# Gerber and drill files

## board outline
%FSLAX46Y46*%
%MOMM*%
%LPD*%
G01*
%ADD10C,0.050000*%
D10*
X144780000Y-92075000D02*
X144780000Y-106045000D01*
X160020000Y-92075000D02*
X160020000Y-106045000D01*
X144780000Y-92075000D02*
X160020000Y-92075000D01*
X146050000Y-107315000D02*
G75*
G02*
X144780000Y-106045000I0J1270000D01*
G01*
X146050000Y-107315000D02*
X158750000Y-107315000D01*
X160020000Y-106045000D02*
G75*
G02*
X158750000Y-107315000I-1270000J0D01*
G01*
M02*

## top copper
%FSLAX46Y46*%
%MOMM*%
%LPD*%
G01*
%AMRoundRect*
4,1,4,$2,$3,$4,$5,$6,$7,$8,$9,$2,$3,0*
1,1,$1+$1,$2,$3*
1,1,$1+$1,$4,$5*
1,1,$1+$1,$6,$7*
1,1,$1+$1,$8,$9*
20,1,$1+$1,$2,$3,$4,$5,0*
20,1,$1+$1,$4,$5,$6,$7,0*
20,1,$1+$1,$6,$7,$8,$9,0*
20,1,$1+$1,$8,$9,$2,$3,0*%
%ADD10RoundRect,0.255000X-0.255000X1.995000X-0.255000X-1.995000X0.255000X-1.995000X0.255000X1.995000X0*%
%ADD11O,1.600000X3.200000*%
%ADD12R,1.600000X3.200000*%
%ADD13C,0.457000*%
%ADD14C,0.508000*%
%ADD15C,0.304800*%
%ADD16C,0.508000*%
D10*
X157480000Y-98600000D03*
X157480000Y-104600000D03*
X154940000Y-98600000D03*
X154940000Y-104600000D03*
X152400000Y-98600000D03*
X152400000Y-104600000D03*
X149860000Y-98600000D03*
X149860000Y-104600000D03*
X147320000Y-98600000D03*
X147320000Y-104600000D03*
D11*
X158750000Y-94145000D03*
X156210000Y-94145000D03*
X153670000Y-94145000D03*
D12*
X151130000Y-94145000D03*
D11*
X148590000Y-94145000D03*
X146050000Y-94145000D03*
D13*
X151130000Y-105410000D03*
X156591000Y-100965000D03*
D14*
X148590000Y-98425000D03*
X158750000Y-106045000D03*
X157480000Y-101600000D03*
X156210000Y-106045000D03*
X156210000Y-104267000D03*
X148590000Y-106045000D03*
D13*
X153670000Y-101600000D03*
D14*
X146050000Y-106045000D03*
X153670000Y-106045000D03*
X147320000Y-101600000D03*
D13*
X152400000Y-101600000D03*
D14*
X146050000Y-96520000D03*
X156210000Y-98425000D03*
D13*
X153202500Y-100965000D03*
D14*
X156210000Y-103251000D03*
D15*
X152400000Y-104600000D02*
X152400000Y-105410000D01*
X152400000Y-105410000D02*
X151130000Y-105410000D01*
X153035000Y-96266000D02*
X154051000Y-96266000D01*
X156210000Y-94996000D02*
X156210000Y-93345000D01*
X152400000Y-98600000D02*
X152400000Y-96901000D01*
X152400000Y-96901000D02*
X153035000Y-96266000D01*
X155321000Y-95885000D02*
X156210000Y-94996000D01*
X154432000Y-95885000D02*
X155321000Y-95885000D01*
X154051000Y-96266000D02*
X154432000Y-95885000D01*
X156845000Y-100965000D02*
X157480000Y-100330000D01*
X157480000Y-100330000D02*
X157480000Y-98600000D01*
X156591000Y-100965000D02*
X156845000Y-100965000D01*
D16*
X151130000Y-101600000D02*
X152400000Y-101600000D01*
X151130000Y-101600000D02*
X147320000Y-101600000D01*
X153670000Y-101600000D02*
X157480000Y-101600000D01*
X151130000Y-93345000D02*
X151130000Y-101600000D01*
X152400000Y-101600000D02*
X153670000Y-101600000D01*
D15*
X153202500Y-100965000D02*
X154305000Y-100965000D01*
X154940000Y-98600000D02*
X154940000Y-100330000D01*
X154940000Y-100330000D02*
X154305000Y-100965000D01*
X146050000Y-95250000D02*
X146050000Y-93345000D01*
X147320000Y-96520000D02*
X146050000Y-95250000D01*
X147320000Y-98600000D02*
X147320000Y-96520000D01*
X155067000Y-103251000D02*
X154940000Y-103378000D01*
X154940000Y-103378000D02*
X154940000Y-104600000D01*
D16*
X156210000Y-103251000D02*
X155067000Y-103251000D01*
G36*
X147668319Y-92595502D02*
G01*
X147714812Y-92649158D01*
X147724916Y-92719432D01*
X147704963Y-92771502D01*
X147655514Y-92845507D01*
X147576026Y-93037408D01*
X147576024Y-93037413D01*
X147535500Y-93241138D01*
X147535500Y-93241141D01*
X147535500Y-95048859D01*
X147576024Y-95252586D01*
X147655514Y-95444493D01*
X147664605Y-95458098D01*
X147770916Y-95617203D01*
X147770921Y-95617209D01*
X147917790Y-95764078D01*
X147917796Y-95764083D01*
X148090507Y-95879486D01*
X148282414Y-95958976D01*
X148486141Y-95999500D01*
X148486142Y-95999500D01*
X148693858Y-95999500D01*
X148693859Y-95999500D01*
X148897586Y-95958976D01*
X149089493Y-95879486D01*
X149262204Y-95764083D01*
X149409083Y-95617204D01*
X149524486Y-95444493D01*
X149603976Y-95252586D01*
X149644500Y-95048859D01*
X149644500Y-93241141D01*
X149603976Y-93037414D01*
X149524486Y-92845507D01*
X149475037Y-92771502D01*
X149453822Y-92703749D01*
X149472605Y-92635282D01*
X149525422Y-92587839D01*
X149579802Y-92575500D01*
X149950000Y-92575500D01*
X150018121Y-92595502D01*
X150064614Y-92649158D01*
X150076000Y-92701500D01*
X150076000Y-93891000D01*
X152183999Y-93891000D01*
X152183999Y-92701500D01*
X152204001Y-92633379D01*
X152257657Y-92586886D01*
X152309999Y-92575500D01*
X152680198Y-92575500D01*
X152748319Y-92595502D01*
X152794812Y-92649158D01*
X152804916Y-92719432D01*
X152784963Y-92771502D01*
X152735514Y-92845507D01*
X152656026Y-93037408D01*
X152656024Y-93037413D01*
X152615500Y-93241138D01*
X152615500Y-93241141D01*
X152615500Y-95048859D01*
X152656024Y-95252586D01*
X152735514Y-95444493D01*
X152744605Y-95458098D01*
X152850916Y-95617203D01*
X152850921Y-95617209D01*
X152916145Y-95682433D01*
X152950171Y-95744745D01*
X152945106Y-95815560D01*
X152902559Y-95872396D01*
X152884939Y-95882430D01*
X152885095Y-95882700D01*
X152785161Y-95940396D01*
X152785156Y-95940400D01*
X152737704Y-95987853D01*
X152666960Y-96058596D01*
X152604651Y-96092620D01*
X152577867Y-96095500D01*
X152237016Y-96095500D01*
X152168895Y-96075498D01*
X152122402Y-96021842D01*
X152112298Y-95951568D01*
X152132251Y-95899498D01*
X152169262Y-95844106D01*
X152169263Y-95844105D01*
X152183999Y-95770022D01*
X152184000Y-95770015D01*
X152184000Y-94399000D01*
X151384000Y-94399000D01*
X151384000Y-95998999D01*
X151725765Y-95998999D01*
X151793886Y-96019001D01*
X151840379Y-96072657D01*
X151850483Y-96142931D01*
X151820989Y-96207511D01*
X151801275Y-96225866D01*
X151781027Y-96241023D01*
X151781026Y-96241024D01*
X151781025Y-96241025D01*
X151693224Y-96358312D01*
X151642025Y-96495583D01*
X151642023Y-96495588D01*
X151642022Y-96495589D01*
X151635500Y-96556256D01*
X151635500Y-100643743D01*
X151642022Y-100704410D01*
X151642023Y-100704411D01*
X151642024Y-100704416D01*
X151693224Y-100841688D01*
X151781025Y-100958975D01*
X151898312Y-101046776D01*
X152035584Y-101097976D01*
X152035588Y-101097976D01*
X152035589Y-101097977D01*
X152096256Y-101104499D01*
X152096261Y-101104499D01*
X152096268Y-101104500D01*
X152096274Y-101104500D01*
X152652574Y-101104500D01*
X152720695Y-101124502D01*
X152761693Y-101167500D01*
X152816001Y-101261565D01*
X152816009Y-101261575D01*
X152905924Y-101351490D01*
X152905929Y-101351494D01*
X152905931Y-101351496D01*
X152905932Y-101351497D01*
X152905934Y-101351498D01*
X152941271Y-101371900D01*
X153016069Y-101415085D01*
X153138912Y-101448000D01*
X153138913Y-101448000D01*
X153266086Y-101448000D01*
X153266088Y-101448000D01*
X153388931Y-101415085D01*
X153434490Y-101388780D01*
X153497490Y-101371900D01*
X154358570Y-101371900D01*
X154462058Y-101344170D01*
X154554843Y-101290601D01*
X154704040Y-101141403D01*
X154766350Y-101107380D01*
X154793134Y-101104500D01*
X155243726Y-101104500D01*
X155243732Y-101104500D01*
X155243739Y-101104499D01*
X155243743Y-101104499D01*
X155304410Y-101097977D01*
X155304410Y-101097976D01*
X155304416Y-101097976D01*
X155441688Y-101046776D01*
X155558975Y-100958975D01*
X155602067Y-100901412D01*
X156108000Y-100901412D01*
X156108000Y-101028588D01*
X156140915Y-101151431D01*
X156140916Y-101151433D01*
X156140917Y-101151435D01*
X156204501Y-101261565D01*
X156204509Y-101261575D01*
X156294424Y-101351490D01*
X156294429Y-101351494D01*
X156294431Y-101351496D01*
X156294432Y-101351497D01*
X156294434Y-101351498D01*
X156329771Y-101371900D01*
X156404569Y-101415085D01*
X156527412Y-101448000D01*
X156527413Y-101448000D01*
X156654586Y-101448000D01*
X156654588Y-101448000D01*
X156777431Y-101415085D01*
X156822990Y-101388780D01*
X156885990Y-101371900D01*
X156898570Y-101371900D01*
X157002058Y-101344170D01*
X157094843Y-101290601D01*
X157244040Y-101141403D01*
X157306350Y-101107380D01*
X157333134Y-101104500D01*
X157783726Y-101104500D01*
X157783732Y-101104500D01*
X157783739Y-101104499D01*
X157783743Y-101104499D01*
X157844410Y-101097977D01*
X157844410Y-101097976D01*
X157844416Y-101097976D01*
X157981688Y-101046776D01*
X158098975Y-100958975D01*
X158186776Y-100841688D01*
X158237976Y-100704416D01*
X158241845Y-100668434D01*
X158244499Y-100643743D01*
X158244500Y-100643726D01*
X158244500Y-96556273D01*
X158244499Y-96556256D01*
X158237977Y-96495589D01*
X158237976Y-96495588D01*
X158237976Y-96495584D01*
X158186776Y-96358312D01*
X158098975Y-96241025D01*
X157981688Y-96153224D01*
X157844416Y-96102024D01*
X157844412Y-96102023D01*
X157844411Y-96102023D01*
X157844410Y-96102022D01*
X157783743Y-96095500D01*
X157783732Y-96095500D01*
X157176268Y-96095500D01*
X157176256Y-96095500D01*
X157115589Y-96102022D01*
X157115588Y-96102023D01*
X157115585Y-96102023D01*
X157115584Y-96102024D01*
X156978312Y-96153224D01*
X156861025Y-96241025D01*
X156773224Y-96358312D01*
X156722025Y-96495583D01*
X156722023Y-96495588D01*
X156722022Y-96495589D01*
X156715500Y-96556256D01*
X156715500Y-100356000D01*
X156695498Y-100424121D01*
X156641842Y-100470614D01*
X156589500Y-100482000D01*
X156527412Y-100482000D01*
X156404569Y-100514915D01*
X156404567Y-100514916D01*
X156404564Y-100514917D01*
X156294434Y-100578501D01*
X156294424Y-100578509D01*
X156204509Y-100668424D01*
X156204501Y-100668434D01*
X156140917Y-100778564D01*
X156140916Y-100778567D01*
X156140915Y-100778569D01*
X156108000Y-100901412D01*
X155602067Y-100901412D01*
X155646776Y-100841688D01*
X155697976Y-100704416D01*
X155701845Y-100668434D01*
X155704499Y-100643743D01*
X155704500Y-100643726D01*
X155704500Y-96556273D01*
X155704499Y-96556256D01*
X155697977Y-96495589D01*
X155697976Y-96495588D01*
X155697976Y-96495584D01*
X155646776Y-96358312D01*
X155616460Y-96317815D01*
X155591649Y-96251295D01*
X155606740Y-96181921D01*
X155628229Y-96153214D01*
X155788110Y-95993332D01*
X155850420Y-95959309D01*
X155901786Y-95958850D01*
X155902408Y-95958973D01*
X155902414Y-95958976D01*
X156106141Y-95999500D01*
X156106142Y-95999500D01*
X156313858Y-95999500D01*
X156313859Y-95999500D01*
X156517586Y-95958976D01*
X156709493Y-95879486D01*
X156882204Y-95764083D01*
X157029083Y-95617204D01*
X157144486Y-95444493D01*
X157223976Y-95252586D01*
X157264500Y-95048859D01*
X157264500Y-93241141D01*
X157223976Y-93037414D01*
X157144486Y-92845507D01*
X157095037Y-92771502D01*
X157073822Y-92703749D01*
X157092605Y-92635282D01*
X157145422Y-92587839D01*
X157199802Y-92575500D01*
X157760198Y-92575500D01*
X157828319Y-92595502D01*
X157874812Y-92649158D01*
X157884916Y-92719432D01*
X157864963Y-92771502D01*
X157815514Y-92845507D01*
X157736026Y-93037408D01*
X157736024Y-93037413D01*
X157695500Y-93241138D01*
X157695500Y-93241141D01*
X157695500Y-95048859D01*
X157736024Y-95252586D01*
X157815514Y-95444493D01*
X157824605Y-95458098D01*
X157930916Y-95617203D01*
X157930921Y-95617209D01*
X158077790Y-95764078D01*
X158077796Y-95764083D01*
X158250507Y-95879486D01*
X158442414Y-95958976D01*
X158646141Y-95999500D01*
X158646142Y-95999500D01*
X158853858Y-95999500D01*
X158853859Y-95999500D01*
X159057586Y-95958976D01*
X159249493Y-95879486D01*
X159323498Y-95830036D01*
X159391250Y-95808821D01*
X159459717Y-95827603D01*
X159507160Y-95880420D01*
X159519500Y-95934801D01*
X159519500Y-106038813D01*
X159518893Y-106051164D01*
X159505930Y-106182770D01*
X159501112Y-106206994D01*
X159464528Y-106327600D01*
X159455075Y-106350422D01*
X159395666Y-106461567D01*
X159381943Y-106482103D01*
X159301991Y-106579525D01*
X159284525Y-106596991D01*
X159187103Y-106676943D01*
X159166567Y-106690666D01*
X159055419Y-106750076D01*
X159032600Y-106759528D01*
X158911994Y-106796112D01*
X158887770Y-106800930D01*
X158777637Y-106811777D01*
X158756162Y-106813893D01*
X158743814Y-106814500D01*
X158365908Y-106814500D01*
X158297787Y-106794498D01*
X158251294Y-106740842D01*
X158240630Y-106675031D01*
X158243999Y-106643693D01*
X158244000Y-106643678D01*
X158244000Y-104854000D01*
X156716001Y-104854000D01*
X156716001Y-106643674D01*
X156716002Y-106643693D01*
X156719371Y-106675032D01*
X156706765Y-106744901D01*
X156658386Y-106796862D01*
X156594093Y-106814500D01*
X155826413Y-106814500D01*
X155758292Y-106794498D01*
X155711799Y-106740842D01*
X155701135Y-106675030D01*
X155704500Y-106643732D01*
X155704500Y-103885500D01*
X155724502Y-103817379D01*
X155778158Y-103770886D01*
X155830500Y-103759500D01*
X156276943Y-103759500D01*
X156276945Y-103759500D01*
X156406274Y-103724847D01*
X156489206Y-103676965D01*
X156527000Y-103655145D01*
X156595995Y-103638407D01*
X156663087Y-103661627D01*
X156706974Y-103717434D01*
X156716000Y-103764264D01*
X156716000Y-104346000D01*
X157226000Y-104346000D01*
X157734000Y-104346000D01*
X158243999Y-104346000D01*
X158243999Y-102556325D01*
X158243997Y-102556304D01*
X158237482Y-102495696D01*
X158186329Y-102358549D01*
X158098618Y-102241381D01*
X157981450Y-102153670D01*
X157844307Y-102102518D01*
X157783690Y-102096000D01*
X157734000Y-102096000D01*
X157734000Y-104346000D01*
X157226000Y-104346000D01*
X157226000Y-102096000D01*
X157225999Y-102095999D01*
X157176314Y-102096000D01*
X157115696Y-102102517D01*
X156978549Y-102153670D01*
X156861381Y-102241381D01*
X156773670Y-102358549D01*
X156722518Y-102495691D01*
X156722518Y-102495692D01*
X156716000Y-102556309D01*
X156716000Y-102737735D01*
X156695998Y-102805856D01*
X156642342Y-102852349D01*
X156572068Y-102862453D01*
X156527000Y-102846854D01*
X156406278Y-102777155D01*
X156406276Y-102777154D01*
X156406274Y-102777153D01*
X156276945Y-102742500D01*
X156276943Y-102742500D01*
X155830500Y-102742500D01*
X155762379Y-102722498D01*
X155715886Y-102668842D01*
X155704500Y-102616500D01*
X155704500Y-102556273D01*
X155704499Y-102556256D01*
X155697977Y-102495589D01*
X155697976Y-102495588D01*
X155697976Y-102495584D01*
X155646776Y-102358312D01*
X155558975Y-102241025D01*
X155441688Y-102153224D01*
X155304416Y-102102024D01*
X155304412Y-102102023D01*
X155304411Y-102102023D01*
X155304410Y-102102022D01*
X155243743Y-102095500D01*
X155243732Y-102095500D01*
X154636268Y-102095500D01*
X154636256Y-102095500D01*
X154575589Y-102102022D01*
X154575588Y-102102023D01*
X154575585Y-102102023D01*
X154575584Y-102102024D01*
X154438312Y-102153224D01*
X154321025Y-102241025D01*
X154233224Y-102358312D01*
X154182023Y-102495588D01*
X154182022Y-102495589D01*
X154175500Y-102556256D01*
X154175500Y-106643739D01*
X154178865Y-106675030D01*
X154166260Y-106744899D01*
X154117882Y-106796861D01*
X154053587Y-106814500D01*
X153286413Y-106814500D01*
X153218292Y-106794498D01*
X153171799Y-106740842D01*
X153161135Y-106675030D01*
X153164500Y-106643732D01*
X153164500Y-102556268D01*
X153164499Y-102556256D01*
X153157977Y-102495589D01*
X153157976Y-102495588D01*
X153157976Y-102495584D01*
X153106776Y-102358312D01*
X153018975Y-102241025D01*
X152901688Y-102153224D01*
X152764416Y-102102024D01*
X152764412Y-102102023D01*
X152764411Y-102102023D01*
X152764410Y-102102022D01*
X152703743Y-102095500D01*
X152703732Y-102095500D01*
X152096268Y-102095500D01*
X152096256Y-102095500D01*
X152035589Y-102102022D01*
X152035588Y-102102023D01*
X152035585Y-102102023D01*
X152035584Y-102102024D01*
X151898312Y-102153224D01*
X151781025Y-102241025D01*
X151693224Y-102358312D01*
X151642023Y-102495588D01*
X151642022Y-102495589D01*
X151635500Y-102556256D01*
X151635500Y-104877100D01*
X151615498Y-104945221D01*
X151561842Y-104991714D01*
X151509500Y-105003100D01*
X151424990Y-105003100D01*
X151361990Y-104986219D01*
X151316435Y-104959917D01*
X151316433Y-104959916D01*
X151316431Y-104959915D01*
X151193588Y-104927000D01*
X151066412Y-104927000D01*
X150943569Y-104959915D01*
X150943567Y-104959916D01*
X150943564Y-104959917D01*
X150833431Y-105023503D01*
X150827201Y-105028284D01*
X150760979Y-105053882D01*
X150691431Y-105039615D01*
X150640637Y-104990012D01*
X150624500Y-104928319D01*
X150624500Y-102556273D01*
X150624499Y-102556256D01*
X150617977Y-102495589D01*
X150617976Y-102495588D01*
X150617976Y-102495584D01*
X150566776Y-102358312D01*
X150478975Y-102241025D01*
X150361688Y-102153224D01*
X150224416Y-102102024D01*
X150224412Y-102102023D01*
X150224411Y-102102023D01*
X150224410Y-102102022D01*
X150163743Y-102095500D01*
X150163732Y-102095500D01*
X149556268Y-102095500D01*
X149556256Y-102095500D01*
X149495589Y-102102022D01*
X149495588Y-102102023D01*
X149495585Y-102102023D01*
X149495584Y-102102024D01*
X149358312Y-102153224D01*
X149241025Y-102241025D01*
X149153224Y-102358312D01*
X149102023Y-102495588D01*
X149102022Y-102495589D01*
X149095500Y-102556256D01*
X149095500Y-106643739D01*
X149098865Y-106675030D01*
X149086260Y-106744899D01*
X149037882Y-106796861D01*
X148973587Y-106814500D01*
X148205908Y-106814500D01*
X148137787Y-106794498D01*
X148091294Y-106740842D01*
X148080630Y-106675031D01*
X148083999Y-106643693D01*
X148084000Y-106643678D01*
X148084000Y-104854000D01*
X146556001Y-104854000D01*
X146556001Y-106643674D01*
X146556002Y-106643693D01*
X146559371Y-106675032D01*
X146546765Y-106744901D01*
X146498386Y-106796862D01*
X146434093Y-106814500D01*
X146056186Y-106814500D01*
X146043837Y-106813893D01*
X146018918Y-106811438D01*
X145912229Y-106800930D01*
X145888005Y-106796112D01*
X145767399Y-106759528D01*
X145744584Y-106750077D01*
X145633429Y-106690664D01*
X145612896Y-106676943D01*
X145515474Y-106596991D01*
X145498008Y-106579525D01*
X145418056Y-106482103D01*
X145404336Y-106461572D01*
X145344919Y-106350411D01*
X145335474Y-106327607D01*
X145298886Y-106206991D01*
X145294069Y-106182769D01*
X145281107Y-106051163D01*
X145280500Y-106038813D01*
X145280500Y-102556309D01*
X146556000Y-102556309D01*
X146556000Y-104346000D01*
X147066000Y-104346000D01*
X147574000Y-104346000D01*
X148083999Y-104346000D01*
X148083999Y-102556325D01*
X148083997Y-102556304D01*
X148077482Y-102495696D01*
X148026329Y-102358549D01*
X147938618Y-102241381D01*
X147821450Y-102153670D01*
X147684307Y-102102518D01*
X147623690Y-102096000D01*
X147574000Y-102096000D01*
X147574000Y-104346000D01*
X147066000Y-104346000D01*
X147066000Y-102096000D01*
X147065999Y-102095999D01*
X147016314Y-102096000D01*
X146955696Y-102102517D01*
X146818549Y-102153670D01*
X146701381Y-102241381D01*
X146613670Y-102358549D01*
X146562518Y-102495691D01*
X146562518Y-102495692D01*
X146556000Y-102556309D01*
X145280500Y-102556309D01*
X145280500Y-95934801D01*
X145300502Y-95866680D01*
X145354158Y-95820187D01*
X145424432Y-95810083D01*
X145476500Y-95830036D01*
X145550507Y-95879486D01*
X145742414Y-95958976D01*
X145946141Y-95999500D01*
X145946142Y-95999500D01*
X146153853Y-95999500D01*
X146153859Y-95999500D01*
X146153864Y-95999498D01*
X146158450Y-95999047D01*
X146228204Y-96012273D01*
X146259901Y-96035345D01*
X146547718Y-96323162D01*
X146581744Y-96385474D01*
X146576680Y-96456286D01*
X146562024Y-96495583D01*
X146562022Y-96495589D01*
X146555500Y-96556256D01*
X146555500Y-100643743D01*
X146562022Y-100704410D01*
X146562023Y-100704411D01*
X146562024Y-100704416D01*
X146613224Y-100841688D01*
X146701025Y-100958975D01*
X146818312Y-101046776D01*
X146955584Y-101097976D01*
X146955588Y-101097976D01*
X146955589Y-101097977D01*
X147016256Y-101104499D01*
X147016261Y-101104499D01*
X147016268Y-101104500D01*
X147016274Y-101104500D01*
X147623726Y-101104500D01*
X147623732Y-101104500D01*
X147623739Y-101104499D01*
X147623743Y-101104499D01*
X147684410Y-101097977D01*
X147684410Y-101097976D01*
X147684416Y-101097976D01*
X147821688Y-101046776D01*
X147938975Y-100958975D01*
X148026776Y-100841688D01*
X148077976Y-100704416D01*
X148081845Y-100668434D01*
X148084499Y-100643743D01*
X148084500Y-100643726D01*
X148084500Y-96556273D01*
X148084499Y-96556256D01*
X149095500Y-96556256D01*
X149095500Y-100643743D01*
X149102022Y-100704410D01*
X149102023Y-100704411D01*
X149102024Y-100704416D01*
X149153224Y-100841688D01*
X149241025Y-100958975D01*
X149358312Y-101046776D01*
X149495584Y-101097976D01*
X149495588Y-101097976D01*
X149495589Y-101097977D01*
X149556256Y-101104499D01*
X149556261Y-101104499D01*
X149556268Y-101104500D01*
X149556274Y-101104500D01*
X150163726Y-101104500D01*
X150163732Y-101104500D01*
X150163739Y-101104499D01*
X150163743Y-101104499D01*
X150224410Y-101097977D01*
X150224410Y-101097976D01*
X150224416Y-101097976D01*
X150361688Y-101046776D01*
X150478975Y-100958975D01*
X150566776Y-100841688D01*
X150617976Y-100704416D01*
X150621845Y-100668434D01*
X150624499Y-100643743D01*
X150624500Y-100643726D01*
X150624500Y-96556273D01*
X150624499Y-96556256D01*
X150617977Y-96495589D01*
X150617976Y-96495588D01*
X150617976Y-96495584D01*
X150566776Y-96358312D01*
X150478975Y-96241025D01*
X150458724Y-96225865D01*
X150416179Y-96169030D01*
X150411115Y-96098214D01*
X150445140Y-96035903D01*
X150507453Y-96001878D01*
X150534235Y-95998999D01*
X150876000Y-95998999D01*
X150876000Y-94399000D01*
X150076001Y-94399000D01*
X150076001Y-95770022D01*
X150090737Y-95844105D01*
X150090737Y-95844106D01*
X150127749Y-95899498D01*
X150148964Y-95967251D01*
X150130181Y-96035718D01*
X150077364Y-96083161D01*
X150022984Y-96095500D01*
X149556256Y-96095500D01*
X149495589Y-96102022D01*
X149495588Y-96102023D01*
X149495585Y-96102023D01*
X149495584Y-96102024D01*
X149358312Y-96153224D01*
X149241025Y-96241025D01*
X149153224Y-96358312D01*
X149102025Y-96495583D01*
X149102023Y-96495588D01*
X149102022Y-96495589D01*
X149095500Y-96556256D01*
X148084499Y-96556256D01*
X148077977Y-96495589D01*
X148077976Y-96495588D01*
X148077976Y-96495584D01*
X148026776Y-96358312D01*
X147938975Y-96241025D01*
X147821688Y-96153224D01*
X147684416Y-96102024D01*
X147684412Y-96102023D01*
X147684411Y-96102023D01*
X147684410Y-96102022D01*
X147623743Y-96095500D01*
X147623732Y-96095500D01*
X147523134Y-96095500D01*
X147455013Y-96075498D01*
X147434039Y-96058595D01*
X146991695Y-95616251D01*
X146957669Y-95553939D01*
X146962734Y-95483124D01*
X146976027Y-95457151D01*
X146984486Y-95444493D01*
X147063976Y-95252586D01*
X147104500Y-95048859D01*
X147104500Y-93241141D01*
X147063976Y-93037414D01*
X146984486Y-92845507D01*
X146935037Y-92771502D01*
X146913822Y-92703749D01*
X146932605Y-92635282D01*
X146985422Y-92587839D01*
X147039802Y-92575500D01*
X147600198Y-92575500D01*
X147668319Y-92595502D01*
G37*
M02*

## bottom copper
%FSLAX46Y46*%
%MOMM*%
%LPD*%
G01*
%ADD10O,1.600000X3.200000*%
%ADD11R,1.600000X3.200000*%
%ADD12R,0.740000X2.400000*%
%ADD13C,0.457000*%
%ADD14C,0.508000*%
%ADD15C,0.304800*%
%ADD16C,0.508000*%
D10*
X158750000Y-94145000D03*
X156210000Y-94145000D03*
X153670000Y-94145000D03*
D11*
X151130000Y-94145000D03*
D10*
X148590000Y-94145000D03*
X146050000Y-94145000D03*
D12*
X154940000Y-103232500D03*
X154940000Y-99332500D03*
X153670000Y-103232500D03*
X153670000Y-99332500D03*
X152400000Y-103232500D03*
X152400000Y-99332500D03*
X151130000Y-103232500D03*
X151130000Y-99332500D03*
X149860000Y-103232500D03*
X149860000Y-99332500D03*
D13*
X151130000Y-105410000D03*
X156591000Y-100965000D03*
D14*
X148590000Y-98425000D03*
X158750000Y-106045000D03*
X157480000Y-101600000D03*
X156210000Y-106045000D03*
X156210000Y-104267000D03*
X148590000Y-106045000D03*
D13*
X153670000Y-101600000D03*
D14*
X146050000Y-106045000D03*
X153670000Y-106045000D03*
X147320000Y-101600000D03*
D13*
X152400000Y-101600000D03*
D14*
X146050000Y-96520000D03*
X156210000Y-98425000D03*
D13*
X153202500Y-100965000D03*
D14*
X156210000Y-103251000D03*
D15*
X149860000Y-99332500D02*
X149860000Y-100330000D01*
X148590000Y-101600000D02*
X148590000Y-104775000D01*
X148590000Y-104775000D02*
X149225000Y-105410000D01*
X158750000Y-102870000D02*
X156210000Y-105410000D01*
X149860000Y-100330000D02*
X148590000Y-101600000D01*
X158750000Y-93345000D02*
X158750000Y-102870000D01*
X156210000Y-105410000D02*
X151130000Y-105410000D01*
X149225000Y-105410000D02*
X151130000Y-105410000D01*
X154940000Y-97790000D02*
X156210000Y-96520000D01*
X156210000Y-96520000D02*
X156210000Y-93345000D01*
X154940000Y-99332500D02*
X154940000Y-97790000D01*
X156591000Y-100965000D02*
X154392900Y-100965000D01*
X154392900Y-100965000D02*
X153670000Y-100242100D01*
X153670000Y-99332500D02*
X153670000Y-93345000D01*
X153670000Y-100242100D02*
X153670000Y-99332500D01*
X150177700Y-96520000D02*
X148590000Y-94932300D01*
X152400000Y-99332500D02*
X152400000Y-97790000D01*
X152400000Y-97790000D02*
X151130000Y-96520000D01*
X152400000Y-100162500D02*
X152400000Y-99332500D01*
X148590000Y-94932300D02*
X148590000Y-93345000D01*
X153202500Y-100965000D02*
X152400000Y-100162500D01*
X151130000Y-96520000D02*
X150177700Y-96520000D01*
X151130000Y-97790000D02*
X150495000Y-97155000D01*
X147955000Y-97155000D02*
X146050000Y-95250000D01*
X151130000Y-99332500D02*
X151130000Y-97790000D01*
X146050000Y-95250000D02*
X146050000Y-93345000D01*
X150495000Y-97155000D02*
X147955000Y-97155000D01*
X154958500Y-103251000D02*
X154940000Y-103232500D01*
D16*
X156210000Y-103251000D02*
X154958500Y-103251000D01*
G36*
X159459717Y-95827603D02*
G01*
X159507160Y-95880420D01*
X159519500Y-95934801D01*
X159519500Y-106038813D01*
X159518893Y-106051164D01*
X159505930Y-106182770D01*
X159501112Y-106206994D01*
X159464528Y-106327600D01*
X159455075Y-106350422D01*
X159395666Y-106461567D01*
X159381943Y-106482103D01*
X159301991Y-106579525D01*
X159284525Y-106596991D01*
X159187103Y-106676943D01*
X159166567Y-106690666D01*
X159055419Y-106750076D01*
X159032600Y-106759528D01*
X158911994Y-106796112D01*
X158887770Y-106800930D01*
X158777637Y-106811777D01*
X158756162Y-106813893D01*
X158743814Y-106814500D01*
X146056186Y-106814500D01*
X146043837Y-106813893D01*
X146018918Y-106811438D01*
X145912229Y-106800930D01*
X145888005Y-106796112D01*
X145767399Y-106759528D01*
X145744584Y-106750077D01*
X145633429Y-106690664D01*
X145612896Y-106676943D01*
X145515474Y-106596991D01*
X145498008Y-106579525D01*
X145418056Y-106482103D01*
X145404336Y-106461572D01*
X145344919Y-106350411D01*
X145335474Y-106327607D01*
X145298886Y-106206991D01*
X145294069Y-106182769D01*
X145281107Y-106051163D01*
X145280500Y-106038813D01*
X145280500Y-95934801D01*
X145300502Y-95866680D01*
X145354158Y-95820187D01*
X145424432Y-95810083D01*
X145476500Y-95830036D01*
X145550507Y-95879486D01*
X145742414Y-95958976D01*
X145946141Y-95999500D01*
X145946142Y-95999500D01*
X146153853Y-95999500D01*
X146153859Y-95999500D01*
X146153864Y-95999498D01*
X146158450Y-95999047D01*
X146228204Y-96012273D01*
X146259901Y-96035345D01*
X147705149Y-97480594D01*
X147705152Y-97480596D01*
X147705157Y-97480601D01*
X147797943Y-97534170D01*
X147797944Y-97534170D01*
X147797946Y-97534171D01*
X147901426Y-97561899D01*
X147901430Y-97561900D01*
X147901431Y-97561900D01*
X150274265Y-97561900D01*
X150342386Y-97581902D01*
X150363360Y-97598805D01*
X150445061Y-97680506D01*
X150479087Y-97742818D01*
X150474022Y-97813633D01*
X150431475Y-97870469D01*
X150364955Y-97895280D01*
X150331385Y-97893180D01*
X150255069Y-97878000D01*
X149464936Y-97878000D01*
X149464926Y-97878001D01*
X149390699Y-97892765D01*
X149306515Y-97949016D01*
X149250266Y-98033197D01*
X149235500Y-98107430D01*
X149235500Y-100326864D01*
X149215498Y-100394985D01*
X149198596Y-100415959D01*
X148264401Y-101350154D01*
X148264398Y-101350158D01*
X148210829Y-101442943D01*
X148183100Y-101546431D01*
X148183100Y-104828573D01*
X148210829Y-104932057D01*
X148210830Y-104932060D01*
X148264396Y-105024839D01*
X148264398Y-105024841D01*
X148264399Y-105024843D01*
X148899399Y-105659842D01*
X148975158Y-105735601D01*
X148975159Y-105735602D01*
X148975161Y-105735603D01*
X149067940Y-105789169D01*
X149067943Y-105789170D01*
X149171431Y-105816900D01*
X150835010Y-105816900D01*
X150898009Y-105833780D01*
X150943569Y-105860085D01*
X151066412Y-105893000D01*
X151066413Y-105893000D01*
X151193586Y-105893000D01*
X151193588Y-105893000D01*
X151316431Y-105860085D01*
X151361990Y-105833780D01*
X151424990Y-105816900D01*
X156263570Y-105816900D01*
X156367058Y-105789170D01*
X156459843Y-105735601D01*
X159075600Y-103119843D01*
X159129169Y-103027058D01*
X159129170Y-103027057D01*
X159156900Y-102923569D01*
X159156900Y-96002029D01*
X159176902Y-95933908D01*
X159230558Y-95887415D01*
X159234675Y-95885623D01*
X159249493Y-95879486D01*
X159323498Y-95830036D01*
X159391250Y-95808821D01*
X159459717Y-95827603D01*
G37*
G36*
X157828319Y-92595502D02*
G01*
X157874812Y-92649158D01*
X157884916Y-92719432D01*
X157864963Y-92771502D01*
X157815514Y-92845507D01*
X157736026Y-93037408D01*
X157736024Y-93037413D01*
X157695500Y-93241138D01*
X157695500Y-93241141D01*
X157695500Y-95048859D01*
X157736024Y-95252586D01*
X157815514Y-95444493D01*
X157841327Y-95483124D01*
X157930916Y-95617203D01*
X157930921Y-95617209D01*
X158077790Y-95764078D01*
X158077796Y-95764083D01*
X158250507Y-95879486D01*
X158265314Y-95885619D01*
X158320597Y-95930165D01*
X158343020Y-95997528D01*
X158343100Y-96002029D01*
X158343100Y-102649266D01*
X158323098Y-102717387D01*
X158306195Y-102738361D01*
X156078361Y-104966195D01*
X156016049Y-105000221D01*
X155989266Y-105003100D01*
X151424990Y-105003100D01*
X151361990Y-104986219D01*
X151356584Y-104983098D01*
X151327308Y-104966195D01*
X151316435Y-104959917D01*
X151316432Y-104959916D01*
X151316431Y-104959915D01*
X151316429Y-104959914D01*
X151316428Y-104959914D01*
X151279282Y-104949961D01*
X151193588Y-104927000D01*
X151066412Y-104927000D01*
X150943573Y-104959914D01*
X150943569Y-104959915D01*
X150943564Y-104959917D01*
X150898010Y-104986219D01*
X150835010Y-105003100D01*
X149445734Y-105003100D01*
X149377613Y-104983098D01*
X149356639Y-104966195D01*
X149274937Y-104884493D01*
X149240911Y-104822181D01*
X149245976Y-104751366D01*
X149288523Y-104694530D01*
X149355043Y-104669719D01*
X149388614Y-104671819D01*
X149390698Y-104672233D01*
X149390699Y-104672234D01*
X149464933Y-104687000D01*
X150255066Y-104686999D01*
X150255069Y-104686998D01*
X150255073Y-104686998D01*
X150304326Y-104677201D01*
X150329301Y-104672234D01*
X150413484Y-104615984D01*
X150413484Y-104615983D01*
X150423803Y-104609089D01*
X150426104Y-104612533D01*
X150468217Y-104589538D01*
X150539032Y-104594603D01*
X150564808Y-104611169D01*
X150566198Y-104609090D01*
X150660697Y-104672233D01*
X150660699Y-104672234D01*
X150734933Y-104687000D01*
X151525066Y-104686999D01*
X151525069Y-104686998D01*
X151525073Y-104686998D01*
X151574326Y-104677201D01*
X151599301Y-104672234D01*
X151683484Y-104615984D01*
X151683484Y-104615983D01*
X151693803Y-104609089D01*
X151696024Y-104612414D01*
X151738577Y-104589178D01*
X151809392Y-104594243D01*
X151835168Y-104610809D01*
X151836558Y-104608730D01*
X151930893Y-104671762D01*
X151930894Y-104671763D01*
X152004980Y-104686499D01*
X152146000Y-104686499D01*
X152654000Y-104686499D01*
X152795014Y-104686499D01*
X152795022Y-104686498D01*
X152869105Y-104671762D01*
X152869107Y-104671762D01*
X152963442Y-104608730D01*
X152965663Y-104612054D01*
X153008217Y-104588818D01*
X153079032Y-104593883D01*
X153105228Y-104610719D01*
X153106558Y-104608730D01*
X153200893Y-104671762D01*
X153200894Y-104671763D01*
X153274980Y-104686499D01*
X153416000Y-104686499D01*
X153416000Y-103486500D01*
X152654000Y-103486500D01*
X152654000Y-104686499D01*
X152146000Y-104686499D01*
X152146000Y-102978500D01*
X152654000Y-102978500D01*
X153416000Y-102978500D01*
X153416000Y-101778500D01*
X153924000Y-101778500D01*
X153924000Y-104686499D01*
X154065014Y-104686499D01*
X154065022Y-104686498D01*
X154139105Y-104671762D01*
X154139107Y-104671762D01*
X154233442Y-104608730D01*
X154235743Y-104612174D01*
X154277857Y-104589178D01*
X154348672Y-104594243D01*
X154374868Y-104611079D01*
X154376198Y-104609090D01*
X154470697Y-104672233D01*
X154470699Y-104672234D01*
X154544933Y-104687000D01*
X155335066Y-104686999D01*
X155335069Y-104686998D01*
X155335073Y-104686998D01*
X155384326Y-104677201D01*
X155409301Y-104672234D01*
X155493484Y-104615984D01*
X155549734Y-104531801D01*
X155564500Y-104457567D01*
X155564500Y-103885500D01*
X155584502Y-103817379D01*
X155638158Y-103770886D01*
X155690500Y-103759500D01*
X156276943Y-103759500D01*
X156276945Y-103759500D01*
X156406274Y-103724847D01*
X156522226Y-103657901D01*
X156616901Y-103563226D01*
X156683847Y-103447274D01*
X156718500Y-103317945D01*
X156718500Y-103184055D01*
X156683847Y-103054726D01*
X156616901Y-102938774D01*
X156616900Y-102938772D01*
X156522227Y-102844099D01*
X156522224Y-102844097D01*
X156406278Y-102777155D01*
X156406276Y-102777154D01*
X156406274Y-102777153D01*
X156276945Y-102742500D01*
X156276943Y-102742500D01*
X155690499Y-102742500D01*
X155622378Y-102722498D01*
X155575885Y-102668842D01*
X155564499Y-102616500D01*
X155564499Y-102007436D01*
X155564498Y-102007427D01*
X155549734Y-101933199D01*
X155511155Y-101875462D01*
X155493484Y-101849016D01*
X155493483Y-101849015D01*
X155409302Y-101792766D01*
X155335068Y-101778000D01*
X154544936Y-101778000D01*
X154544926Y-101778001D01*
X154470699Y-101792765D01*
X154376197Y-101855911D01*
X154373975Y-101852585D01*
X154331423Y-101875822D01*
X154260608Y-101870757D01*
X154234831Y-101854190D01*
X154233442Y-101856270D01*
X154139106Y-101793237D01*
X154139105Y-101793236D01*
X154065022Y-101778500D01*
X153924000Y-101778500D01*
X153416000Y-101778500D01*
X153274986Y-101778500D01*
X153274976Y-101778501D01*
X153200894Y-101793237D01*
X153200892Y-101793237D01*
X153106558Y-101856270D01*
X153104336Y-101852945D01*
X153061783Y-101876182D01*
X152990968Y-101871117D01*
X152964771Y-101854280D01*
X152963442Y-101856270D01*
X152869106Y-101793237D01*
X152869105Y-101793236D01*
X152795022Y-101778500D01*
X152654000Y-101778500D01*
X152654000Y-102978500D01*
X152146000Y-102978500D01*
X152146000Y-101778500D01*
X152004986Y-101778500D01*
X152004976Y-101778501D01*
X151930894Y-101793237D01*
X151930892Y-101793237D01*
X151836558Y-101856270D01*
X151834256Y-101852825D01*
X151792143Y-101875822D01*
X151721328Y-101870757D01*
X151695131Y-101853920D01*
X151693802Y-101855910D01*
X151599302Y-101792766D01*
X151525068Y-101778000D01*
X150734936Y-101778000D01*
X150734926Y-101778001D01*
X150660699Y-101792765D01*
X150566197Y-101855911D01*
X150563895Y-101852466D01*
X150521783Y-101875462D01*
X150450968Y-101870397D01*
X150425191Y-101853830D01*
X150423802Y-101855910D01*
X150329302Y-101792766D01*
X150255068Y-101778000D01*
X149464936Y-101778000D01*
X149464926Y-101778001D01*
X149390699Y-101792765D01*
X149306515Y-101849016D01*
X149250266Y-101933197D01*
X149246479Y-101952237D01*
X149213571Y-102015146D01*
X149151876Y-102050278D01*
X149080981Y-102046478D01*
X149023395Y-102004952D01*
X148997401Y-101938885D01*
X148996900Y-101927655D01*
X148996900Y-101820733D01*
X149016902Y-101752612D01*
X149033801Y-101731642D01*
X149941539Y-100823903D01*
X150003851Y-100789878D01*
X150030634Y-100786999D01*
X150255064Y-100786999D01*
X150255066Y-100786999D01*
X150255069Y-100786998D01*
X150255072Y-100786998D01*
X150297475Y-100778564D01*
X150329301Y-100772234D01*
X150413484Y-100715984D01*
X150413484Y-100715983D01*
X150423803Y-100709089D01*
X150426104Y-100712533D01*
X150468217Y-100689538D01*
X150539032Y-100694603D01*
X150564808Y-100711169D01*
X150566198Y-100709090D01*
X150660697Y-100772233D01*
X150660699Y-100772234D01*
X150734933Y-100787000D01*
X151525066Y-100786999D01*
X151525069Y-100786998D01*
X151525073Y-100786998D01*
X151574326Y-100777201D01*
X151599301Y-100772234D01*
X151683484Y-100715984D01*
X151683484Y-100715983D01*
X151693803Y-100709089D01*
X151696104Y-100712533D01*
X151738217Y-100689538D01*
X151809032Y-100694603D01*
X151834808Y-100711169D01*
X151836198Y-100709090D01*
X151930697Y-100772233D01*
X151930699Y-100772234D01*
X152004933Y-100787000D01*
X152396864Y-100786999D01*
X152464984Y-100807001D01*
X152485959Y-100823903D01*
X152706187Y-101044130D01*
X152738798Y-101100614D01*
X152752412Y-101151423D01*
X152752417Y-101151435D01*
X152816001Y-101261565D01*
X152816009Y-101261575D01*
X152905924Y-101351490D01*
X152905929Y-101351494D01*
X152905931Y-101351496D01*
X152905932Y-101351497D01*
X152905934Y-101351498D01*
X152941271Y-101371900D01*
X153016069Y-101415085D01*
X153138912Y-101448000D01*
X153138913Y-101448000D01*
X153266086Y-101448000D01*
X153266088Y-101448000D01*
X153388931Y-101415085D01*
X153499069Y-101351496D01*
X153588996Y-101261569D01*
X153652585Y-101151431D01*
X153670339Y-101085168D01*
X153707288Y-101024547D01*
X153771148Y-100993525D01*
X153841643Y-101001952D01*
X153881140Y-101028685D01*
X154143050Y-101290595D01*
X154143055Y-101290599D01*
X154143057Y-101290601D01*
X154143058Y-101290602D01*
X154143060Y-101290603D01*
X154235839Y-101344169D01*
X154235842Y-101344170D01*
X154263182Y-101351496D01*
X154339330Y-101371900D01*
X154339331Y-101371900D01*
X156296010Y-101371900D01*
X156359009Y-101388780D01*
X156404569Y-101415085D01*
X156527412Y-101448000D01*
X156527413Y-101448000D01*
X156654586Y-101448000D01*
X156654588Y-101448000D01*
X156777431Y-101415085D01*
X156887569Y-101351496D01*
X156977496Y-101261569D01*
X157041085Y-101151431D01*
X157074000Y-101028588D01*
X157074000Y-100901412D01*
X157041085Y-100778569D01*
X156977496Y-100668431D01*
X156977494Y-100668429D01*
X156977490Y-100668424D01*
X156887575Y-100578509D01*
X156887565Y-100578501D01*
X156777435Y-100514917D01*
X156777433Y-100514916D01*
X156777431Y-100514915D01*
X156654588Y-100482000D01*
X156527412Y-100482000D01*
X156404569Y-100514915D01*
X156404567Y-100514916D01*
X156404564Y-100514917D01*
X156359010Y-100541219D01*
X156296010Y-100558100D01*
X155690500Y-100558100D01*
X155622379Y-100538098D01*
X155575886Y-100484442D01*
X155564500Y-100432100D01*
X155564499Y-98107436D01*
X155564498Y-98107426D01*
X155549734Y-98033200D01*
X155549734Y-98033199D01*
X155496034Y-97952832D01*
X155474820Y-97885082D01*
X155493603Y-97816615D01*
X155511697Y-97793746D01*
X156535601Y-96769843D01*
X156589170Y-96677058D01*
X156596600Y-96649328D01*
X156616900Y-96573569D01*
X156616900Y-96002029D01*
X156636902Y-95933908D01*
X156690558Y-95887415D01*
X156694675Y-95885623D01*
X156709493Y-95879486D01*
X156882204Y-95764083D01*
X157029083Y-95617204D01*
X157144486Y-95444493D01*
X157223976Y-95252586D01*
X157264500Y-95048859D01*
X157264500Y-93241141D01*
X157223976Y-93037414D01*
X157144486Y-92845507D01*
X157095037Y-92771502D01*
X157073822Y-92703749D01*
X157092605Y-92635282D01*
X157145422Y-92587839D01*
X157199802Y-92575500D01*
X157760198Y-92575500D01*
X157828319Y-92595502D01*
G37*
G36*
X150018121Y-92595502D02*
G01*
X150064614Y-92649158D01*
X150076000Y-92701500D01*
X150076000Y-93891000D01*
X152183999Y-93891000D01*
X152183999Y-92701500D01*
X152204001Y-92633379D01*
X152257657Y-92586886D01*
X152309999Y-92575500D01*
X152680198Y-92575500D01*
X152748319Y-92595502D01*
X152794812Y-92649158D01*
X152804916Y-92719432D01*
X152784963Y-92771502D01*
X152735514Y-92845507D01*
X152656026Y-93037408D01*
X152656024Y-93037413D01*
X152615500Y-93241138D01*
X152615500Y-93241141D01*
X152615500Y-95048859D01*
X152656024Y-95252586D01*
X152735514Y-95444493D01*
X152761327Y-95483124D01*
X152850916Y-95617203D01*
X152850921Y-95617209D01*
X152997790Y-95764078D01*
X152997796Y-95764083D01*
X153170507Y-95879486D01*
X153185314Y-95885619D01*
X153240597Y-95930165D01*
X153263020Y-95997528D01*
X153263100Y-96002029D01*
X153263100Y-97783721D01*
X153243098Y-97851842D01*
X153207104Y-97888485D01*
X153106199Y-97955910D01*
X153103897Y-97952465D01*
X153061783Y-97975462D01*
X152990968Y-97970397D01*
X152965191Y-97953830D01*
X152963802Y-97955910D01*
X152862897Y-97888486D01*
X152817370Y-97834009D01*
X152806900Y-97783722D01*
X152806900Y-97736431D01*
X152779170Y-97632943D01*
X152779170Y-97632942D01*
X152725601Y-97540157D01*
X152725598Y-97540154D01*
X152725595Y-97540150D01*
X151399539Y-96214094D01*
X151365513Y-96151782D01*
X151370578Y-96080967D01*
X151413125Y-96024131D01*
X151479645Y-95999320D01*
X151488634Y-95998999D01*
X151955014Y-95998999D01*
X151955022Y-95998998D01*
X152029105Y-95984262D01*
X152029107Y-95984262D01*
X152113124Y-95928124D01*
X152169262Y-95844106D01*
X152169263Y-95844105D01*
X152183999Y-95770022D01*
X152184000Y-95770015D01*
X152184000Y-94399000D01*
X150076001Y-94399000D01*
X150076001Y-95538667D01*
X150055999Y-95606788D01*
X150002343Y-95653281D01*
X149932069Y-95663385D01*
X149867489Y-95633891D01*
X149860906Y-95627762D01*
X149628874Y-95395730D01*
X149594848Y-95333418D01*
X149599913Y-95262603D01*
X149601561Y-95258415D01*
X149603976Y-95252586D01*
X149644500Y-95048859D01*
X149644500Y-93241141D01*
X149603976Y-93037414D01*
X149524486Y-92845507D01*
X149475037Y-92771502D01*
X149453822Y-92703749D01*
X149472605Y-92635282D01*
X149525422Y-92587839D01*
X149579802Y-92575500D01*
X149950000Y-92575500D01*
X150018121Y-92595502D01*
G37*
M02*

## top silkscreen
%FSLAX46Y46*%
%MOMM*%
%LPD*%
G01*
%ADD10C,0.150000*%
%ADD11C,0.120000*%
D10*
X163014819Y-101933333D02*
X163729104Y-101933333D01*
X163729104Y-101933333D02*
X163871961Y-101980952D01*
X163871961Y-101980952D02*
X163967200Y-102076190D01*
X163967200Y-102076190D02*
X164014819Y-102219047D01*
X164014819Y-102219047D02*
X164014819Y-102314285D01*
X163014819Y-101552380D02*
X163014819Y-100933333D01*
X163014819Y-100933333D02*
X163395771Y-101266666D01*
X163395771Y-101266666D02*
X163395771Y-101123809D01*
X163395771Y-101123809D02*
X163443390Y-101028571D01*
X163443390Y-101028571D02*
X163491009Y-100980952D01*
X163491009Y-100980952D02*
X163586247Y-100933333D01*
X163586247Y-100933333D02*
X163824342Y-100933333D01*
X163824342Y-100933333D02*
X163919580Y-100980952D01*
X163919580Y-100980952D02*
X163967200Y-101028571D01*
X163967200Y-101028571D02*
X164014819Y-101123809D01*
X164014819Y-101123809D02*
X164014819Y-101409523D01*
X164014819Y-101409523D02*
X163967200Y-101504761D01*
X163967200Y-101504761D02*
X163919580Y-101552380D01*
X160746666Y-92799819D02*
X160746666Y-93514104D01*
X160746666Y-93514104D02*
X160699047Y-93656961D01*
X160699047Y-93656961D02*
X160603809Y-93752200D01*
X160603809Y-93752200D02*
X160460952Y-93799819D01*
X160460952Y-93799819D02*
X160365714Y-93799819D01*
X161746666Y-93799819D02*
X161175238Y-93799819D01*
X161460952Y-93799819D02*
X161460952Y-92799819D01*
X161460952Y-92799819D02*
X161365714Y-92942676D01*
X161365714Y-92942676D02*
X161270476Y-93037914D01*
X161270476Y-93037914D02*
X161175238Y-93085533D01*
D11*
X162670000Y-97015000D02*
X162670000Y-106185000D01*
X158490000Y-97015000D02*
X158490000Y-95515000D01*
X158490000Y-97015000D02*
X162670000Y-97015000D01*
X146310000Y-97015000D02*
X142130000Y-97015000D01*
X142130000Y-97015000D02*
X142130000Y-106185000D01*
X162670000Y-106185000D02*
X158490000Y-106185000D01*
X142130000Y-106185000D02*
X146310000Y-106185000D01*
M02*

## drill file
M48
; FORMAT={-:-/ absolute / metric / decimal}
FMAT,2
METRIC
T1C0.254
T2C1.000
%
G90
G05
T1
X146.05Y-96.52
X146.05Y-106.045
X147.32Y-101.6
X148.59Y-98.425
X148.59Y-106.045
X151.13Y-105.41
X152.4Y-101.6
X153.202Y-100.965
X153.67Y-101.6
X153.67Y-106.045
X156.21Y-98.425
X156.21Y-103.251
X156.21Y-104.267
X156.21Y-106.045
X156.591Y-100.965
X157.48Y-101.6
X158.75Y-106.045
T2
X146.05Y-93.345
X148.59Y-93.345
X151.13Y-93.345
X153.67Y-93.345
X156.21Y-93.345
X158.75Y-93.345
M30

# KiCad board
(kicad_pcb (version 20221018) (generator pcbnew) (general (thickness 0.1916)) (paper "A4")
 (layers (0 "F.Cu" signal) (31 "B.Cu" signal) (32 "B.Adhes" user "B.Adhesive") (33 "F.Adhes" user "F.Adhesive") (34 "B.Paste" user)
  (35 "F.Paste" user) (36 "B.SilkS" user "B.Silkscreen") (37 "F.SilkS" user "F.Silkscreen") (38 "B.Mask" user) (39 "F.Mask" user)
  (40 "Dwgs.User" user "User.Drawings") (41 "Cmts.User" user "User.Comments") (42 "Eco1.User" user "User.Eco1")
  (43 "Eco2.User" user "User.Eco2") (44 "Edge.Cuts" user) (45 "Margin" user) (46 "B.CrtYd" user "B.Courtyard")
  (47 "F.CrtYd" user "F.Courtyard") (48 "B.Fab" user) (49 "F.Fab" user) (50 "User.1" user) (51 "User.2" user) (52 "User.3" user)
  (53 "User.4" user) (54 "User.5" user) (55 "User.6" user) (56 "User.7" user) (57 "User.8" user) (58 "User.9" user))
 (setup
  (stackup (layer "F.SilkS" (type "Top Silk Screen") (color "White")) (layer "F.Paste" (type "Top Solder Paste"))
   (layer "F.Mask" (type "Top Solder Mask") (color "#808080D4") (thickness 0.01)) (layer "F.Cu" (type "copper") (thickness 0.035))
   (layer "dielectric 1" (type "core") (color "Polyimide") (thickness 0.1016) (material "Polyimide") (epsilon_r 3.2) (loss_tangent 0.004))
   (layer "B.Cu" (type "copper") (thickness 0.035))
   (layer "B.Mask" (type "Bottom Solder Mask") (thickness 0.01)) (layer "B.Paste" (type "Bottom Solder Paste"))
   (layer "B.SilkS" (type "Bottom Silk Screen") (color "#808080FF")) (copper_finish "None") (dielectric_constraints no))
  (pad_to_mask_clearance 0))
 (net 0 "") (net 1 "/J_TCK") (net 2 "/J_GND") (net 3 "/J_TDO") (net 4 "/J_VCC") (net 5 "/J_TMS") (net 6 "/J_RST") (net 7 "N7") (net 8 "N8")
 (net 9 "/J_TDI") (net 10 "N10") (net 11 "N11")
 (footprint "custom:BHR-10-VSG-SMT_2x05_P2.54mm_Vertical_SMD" (layer "F.Cu") (at 152.4 101.6 -90)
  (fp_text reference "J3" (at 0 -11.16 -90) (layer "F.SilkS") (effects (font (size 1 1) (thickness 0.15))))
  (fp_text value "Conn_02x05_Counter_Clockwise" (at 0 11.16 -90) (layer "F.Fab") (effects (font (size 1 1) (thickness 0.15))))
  (fp_line (start -4.585 -10.27) (end 4.585 -10.27) (stroke (width 0.12) (type solid)) (layer "F.SilkS"))
  (fp_line (start -4.585 -6.09) (end -6.085 -6.09) (stroke (width 0.12) (type solid)) (layer "F.SilkS"))
  (fp_line (start -4.585 -6.09) (end -4.585 -10.27) (stroke (width 0.12) (type solid)) (layer "F.SilkS"))
  (fp_line (start -4.585 6.09) (end -4.585 10.27) (stroke (width 0.12) (type solid)) (layer "F.SilkS"))
  (fp_line (start -4.585 10.27) (end 4.585 10.27) (stroke (width 0.12) (type solid)) (layer "F.SilkS"))
  (fp_line (start 4.585 -10.27) (end 4.585 -6.09) (stroke (width 0.12) (type solid)) (layer "F.SilkS"))
  (fp_line (start 4.585 10.27) (end 4.585 6.09) (stroke (width 0.12) (type solid)) (layer "F.SilkS"))
  (pad "1" smd roundrect (at -3 -5.08 270) (size 4.5 1.02) (layers "F.Cu" "F.Paste" "F.Mask") (roundrect_rratio 0.25) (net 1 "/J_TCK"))
  (pad "2" smd roundrect (at 3 -5.08 270) (size 4.5 1.02) (layers "F.Cu" "F.Paste" "F.Mask") (roundrect_rratio 0.25) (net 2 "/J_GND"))
  (pad "3" smd roundrect (at -3 -2.54 270) (size 4.5 1.02) (layers "F.Cu" "F.Paste" "F.Mask") (roundrect_rratio 0.25) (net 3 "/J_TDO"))
  (pad "4" smd roundrect (at 3 -2.54 270) (size 4.5 1.02) (layers "F.Cu" "F.Paste" "F.Mask") (roundrect_rratio 0.25) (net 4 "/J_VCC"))
  (pad "5" smd roundrect (at -3 0 270) (size 4.5 1.02) (layers "F.Cu" "F.Paste" "F.Mask") (roundrect_rratio 0.25) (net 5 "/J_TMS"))
  (pad "6" smd roundrect (at 3 0 270) (size 4.5 1.02) (layers "F.Cu" "F.Paste" "F.Mask") (roundrect_rratio 0.25) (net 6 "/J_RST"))
  (pad "7" smd roundrect (at -3 2.54 270) (size 4.5 1.02) (layers "F.Cu" "F.Paste" "F.Mask") (roundrect_rratio 0.25) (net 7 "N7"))
  (pad "8" smd roundrect (at 3 2.54 270) (size 4.5 1.02) (layers "F.Cu" "F.Paste" "F.Mask") (roundrect_rratio 0.25) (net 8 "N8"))
  (pad "9" smd roundrect (at -3 5.08 270) (size 4.5 1.02) (layers "F.Cu" "F.Paste" "F.Mask") (roundrect_rratio 0.25) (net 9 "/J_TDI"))
  (pad "10" smd roundrect (at 3 5.08 270) (size 4.5 1.02) (layers "F.Cu" "F.Paste" "F.Mask") (roundrect_rratio 0.25) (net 2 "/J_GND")))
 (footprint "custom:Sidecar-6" (layer "F.Cu") (at 158.75 93.345 -90)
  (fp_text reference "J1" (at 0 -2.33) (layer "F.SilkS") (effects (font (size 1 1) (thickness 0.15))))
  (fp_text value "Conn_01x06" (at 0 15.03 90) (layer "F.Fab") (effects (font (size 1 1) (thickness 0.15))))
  (pad "1" thru_hole oval (at 0 0 270) (size 3.2 1.6) (drill 1 (offset 0.8 0)) (layers "*.Cu" "*.Mask") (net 6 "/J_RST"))
  (pad "2" thru_hole oval (at 0 2.54 270) (size 3.2 1.6) (drill 1 (offset 0.8 0)) (layers "*.Cu" "*.Mask") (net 5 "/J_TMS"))
  (pad "3" thru_hole oval (at 0 5.08 270) (size 3.2 1.6) (drill 1 (offset 0.8 0)) (layers "*.Cu" "*.Mask") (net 1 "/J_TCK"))
  (pad "4" thru_hole rect (at 0 7.62 270) (size 3.2 1.6) (drill 1 (offset 0.8 0)) (layers "*.Cu" "*.Mask") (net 2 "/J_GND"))
  (pad "5" thru_hole oval (at 0 10.16 270) (size 3.2 1.6) (drill 1 (offset 0.8 0)) (layers "*.Cu" "*.Mask") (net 3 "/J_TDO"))
  (pad "6" thru_hole oval (at 0 12.7 270) (size 3.2 1.6) (drill 1 (offset 0.8 0)) (layers "*.Cu" "*.Mask") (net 9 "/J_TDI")))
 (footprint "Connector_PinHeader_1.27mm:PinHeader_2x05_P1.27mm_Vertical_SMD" (layer "B.Cu") (at 152.4 101.2825 90)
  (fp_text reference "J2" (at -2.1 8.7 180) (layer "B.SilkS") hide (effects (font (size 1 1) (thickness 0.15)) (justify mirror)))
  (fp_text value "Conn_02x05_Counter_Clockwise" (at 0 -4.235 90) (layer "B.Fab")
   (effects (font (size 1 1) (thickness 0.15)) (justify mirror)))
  (pad "1" smd rect (at -1.95 2.54 90) (size 2.4 0.74) (layers "B.Cu" "B.Paste" "B.Mask") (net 4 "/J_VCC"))
  (pad "2" smd rect (at 1.95 2.54 90) (size 2.4 0.74) (layers "B.Cu" "B.Paste" "B.Mask") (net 5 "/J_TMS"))
  (pad "3" smd rect (at -1.95 1.27 90) (size 2.4 0.74) (layers "B.Cu" "B.Paste" "B.Mask") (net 2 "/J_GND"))
  (pad "4" smd rect (at 1.95 1.27 90) (size 2.4 0.74) (layers "B.Cu" "B.Paste" "B.Mask") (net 1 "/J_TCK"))
  (pad "5" smd rect (at -1.95 0 90) (size 2.4 0.74) (layers "B.Cu" "B.Paste" "B.Mask") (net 2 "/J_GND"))
  (pad "6" smd rect (at 1.95 0 90) (size 2.4 0.74) (layers "B.Cu" "B.Paste" "B.Mask") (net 3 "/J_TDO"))
  (pad "7" smd rect (at -1.95 -1.27 90) (size 2.4 0.74) (layers "B.Cu" "B.Paste" "B.Mask") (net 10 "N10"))
  (pad "8" smd rect (at 1.95 -1.27 90) (size 2.4 0.74) (layers "B.Cu" "B.Paste" "B.Mask") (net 9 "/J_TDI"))
  (pad "9" smd rect (at -1.95 -2.54 90) (size 2.4 0.74) (layers "B.Cu" "B.Paste" "B.Mask") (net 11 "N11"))
  (pad "10" smd rect (at 1.95 -2.54 90) (size 2.4 0.74) (layers "B.Cu" "B.Paste" "B.Mask") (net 6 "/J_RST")))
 (gr_line (start 144.78 92.075) (end 144.78 106.045) (stroke (width 0.05) (type default)) (layer "Edge.Cuts"))
 (gr_line (start 160.02 92.075) (end 160.02 106.045) (stroke (width 0.05) (type default)) (layer "Edge.Cuts"))
 (gr_line (start 144.78 92.075) (end 160.02 92.075) (stroke (width 0.05) (type default)) (layer "Edge.Cuts"))
 (gr_arc (start 146.05 107.315) (mid 145.151974 106.943026) (end 144.78 106.045) (stroke (width 0.05) (type default)) (layer "Edge.Cuts"))
 (gr_line (start 146.05 107.315) (end 158.75 107.315) (stroke (width 0.05) (type default)) (layer "Edge.Cuts"))
 (gr_arc (start 160.02 106.045) (mid 159.648026 106.943026) (end 158.75 107.315) (stroke (width 0.05) (type default)) (layer "Edge.Cuts"))
 (segment (start 152.4 104.6) (end 152.4 105.41) (width 0.3048) (layer "F.Cu") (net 6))
 (segment (start 152.4 105.41) (end 151.13 105.41) (width 0.3048) (layer "F.Cu") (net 6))
 (via (at 151.13 105.41) (size 0.457) (drill 0.254) (layers "F.Cu" "B.Cu") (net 6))
 (segment (start 149.86 99.3325) (end 149.86 100.33) (width 0.3048) (layer "B.Cu") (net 6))
 (segment (start 148.59 101.6) (end 148.59 104.775) (width 0.3048) (layer "B.Cu") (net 6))
 (segment (start 148.59 104.775) (end 149.225 105.41) (width 0.3048) (layer "B.Cu") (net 6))
 (segment (start 158.75 102.87) (end 156.21 105.41) (width 0.3048) (layer "B.Cu") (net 6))
 (segment (start 149.86 100.33) (end 148.59 101.6) (width 0.3048) (layer "B.Cu") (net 6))
 (segment (start 158.75 93.345) (end 158.75 102.87) (width 0.3048) (layer "B.Cu") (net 6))
 (segment (start 156.21 105.41) (end 151.13 105.41) (width 0.3048) (layer "B.Cu") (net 6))
 (segment (start 149.225 105.41) (end 151.13 105.41) (width 0.3048) (layer "B.Cu") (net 6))
 (segment (start 153.035 96.266) (end 154.051 96.266) (width 0.3048) (layer "F.Cu") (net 5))
 (segment (start 156.21 94.996) (end 156.21 93.345) (width 0.3048) (layer "F.Cu") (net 5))
 (segment (start 152.4 98.6) (end 152.4 96.901) (width 0.3048) (layer "F.Cu") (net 5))
 (segment (start 152.4 96.901) (end 153.035 96.266) (width 0.3048) (layer "F.Cu") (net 5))
 (segment (start 155.321 95.885) (end 156.21 94.996) (width 0.3048) (layer "F.Cu") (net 5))
 (segment (start 154.432 95.885) (end 155.321 95.885) (width 0.3048) (layer "F.Cu") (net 5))
 (segment (start 154.051 96.266) (end 154.432 95.885) (width 0.3048) (layer "F.Cu") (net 5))
 (segment (start 154.94 97.79) (end 156.21 96.52) (width 0.3048) (layer "B.Cu") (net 5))
 (segment (start 156.21 96.52) (end 156.21 93.345) (width 0.3048) (layer "B.Cu") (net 5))
 (segment (start 154.94 99.3325) (end 154.94 97.79) (width 0.3048) (layer "B.Cu") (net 5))
 (segment (start 156.845 100.965) (end 157.48 100.33) (width 0.3048) (layer "F.Cu") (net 1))
 (segment (start 157.48 100.33) (end 157.48 98.6) (width 0.3048) (layer "F.Cu") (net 1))
 (segment (start 156.591 100.965) (end 156.845 100.965) (width 0.3048) (layer "F.Cu") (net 1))
 (via (at 156.591 100.965) (size 0.457) (drill 0.254) (layers "F.Cu" "B.Cu") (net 1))
 (segment (start 156.591 100.965) (end 154.3929 100.965) (width 0.3048) (layer "B.Cu") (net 1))
 (segment (start 154.3929 100.965) (end 153.67 100.2421) (width 0.3048) (layer "B.Cu") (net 1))
 (segment (start 153.67 99.3325) (end 153.67 93.345) (width 0.3048) (layer "B.Cu") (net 1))
 (segment (start 153.67 100.2421) (end 153.67 99.3325) (width 0.3048) (layer "B.Cu") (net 1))
 (segment (start 151.13 101.6) (end 152.4 101.6) (width 0.508) (layer "F.Cu") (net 2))
 (segment (start 151.13 101.6) (end 147.32 101.6) (width 0.508) (layer "F.Cu") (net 2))
 (segment (start 153.67 101.6) (end 157.48 101.6) (width 0.508) (layer "F.Cu") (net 2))
 (segment (start 151.13 93.345) (end 151.13 101.6) (width 0.508) (layer "F.Cu") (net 2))
 (segment (start 152.4 101.6) (end 153.67 101.6) (width 0.508) (layer "F.Cu") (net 2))
 (via (at 148.59 98.425) (size 0.508) (drill 0.254) (layers "F.Cu" "B.Cu") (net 2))
 (via (at 158.75 106.045) (size 0.508) (drill 0.254) (layers "F.Cu" "B.Cu") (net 2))
 (via (at 157.48 101.6) (size 0.508) (drill 0.254) (layers "F.Cu" "B.Cu") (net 2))
 (via (at 156.21 106.045) (size 0.508) (drill 0.254) (layers "F.Cu" "B.Cu") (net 2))
 (via (at 156.21 104.267) (size 0.508) (drill 0.254) (layers "F.Cu" "B.Cu") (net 2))
 (via (at 148.59 106.045) (size 0.508) (drill 0.254) (layers "F.Cu" "B.Cu") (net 2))
 (via (at 153.67 101.6) (size 0.457) (drill 0.254) (layers "F.Cu" "B.Cu") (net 2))
 (via (at 146.05 106.045) (size 0.508) (drill 0.254) (layers "F.Cu" "B.Cu") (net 2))
 (via (at 153.67 106.045) (size 0.508) (drill 0.254) (layers "F.Cu" "B.Cu") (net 2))
 (via (at 147.32 101.6) (size 0.508) (drill 0.254) (layers "F.Cu" "B.Cu") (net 2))
 (via (at 152.4 101.6) (size 0.457) (drill 0.254) (layers "F.Cu" "B.Cu") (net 2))
 (via (at 146.05 96.52) (size 0.508) (drill 0.254) (layers "F.Cu" "B.Cu") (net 2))
 (via (at 156.21 98.425) (size 0.508) (drill 0.254) (layers "F.Cu" "B.Cu") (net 2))
 (segment (start 153.2025 100.965) (end 154.305 100.965) (width 0.3048) (layer "F.Cu") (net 3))
 (segment (start 154.94 98.6) (end 154.94 100.33) (width 0.3048) (layer "F.Cu") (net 3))
 (segment (start 154.94 100.33) (end 154.305 100.965) (width 0.3048) (layer "F.Cu") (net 3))
 (via (at 153.2025 100.965) (size 0.457) (drill 0.254) (layers "F.Cu" "B.Cu") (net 3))
 (segment (start 150.1777 96.52) (end 148.59 94.9323) (width 0.3048) (layer "B.Cu") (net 3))
 (segment (start 152.4 99.3325) (end 152.4 97.79) (width 0.3048) (layer "B.Cu") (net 3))
 (segment (start 152.4 97.79) (end 151.13 96.52) (width 0.3048) (layer "B.Cu") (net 3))
 (segment (start 152.4 100.1625) (end 152.4 99.3325) (width 0.3048) (layer "B.Cu") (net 3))
 (segment (start 148.59 94.9323) (end 148.59 93.345) (width 0.3048) (layer "B.Cu") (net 3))
 (segment (start 153.2025 100.965) (end 152.4 100.1625) (width 0.3048) (layer "B.Cu") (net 3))
 (segment (start 151.13 96.52) (end 150.1777 96.52) (width 0.3048) (layer "B.Cu") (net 3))
 (segment (start 146.05 95.25) (end 146.05 93.345) (width 0.3048) (layer "F.Cu") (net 9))
 (segment (start 147.32 96.52) (end 146.05 95.25) (width 0.3048) (layer "F.Cu") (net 9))
 (segment (start 147.32 98.6) (end 147.32 96.52) (width 0.3048) (layer "F.Cu") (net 9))
 (segment (start 151.13 97.79) (end 150.495 97.155) (width 0.3048) (layer "B.Cu") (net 9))
 (segment (start 147.955 97.155) (end 146.05 95.25) (width 0.3048) (layer "B.Cu") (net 9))
 (segment (start 151.13 99.3325) (end 151.13 97.79) (width 0.3048) (layer "B.Cu") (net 9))
 (segment (start 146.05 95.25) (end 146.05 93.345) (width 0.3048) (layer "B.Cu") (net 9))
 (segment (start 150.495 97.155) (end 147.955 97.155) (width 0.3048) (layer "B.Cu") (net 9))
 (segment (start 155.067 103.251) (end 154.94 103.378) (width 0.3048) (layer "F.Cu") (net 4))
 (segment (start 154.94 103.378) (end 154.94 104.6) (width 0.3048) (layer "F.Cu") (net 4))
 (segment (start 156.21 103.251) (end 155.067 103.251) (width 0.508) (layer "F.Cu") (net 4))
 (via (at 156.21 103.251) (size 0.508) (drill 0.254) (layers "F.Cu" "B.Cu") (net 4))
 (segment (start 154.9585 103.251) (end 154.94 103.2325) (width 0.3048) (layer "B.Cu") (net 4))
 (segment (start 156.21 103.251) (end 154.9585 103.251) (width 0.508) (layer "B.Cu") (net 4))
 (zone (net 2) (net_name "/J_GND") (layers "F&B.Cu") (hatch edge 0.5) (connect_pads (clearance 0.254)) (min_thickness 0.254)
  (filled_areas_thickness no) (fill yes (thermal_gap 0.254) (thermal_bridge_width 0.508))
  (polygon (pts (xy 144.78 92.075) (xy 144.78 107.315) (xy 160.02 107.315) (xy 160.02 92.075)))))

